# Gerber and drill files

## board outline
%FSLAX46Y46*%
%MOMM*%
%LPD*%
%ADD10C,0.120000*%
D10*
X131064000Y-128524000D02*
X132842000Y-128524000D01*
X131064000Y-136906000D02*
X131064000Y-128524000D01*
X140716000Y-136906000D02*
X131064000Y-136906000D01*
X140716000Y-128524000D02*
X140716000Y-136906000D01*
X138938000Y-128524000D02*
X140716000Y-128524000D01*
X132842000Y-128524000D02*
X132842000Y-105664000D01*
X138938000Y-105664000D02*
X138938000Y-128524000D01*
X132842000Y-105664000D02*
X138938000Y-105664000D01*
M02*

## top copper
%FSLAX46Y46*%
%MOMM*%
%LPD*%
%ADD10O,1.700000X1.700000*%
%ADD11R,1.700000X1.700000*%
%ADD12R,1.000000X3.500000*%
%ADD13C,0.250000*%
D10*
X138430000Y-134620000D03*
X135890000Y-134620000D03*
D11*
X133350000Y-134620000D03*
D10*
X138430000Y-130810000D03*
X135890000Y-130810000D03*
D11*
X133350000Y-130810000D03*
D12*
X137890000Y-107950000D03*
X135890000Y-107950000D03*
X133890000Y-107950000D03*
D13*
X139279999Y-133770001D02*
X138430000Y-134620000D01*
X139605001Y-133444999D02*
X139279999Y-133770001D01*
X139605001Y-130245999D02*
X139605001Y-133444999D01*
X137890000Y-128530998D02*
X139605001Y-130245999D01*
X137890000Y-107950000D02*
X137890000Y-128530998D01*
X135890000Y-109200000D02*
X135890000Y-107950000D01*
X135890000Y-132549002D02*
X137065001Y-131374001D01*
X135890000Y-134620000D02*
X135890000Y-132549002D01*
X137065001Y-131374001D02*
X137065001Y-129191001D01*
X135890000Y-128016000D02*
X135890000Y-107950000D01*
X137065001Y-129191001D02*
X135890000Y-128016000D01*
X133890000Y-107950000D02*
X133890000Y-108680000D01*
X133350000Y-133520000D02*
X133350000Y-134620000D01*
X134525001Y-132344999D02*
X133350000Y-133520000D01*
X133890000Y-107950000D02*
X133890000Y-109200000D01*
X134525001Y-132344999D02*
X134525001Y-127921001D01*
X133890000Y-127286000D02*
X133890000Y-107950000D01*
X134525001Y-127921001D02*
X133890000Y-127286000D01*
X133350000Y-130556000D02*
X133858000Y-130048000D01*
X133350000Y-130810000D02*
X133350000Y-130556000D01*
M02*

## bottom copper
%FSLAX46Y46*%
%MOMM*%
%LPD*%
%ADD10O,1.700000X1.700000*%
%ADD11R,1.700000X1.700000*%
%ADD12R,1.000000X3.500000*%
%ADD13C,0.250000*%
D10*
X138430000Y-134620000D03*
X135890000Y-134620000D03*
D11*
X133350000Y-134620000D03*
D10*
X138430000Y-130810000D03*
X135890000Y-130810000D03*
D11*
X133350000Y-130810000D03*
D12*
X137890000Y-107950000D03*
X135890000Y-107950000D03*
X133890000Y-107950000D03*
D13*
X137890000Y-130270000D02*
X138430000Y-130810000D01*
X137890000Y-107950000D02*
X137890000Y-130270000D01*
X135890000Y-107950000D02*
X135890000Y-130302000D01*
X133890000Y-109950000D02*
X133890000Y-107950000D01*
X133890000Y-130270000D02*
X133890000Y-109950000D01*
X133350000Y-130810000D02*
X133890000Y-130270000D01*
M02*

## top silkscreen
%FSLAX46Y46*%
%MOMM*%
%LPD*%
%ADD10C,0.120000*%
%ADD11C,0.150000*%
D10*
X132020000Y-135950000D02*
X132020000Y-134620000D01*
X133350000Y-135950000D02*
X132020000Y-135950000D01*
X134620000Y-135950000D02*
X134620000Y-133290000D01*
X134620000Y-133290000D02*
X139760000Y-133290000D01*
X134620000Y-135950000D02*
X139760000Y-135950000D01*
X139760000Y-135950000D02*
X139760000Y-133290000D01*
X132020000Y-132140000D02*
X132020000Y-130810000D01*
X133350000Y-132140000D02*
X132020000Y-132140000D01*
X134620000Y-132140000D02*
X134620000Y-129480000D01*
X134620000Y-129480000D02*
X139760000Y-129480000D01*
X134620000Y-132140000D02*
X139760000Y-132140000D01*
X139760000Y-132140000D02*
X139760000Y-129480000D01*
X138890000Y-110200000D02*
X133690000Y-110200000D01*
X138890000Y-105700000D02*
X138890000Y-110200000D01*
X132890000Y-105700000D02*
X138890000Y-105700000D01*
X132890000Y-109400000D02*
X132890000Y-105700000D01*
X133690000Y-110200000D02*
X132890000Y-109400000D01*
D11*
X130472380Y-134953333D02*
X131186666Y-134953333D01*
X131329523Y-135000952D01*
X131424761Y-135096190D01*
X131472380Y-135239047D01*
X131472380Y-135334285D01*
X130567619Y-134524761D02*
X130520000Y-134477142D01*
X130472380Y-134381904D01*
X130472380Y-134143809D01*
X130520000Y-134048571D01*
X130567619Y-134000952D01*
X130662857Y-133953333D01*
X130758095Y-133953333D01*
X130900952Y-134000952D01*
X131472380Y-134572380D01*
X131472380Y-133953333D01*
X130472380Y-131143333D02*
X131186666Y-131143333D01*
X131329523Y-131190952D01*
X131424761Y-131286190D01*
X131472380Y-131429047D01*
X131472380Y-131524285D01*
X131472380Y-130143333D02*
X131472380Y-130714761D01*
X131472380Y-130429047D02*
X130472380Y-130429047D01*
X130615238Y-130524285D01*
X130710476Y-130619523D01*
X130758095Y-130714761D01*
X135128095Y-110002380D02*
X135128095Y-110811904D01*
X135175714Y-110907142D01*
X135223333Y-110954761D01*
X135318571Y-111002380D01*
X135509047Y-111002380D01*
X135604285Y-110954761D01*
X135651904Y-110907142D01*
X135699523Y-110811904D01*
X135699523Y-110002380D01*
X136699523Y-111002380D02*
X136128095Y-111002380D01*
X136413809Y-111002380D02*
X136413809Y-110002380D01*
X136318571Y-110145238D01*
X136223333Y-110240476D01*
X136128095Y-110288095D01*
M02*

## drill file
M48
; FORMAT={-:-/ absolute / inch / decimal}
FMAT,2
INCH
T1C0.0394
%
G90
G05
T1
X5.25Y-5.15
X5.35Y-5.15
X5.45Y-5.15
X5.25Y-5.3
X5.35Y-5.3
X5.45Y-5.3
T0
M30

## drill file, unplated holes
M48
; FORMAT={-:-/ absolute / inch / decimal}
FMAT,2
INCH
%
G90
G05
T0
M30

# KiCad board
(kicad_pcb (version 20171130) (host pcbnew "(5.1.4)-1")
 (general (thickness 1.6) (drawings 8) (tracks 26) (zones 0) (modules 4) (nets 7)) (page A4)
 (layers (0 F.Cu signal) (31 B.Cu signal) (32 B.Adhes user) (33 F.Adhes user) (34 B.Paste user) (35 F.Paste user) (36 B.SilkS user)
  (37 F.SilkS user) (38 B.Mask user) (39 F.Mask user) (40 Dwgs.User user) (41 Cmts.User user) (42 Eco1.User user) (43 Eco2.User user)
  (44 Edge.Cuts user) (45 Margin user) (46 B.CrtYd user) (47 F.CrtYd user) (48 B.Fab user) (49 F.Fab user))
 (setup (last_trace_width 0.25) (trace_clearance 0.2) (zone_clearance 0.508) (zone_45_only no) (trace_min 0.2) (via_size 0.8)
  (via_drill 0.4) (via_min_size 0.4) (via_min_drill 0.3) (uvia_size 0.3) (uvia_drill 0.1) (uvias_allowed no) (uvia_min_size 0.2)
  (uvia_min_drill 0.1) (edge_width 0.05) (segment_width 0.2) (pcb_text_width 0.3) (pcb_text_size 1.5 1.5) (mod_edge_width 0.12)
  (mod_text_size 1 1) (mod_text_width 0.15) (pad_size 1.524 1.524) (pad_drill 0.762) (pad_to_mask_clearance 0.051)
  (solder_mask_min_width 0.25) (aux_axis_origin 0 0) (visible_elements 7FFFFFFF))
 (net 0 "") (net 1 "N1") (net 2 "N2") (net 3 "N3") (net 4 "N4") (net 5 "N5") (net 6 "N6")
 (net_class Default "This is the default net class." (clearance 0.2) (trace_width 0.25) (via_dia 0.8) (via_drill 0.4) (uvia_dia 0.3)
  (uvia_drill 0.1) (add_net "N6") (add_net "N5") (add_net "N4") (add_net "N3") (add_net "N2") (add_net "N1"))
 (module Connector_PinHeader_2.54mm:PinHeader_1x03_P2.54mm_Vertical (layer F.Cu) (at 133.35 134.62 90)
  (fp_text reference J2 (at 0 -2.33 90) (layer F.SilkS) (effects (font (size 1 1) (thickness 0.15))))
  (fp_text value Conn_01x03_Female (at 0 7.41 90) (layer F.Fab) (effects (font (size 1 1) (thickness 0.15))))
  (fp_line (start -1.33 -1.33) (end 0 -1.33) (layer F.SilkS) (width 0.12))
  (fp_line (start -1.33 0) (end -1.33 -1.33) (layer F.SilkS) (width 0.12))
  (fp_line (start -1.33 1.27) (end 1.33 1.27) (layer F.SilkS) (width 0.12))
  (fp_line (start 1.33 1.27) (end 1.33 6.41) (layer F.SilkS) (width 0.12))
  (fp_line (start -1.33 1.27) (end -1.33 6.41) (layer F.SilkS) (width 0.12))
  (fp_line (start -1.33 6.41) (end 1.33 6.41) (layer F.SilkS) (width 0.12))
  (pad 3 thru_hole oval (at 0 5.08 90) (size 1.7 1.7) (drill 1) (layers *.Cu *.Mask) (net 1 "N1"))
  (pad 2 thru_hole oval (at 0 2.54 90) (size 1.7 1.7) (drill 1) (layers *.Cu *.Mask) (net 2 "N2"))
  (pad 1 thru_hole rect (at 0 0 90) (size 1.7 1.7) (drill 1) (layers *.Cu *.Mask) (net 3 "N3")))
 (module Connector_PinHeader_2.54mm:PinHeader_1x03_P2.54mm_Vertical (layer F.Cu) (at 133.35 130.81 90)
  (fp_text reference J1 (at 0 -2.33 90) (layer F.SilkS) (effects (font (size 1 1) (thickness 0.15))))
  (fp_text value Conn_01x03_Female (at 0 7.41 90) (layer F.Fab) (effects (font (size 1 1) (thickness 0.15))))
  (fp_line (start -1.33 -1.33) (end 0 -1.33) (layer F.SilkS) (width 0.12))
  (fp_line (start -1.33 0) (end -1.33 -1.33) (layer F.SilkS) (width 0.12))
  (fp_line (start -1.33 1.27) (end 1.33 1.27) (layer F.SilkS) (width 0.12))
  (fp_line (start 1.33 1.27) (end 1.33 6.41) (layer F.SilkS) (width 0.12))
  (fp_line (start -1.33 1.27) (end -1.33 6.41) (layer F.SilkS) (width 0.12))
  (fp_line (start -1.33 6.41) (end 1.33 6.41) (layer F.SilkS) (width 0.12))
  (pad 3 thru_hole oval (at 0 5.08 90) (size 1.7 1.7) (drill 1) (layers *.Cu *.Mask) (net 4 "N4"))
  (pad 2 thru_hole oval (at 0 2.54 90) (size 1.7 1.7) (drill 1) (layers *.Cu *.Mask) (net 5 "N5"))
  (pad 1 thru_hole rect (at 0 0 90) (size 1.7 1.7) (drill 1) (layers *.Cu *.Mask) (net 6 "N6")))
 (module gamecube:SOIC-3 (layer B.Cu) (at 135.89 107.95)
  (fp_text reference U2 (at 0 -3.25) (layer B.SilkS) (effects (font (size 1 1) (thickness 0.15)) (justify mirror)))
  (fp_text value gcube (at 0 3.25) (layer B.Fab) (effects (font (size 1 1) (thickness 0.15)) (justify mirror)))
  (pad 3 smd rect (at 2 0) (size 1 3.5) (layers B.Cu B.Paste B.Mask) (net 4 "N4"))
  (pad 2 smd rect (at 0 0) (size 1 3.5) (layers B.Cu B.Paste B.Mask) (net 5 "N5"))
  (pad 1 smd rect (at -2 0) (size 1 3.5) (layers B.Cu B.Paste B.Mask) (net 6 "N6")))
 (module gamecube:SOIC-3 (layer F.Cu) (at 135.89 107.95)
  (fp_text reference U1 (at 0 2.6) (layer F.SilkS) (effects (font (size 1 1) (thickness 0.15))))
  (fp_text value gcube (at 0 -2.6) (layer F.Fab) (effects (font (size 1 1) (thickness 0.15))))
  (fp_line (start 3 2.25) (end -2.2 2.25) (layer F.SilkS) (width 0.12))
  (fp_line (start 3 -2.25) (end 3 2.25) (layer F.SilkS) (width 0.12))
  (fp_line (start -3 -2.25) (end 3 -2.25) (layer F.SilkS) (width 0.12))
  (fp_line (start -3 1.45) (end -3 -2.25) (layer F.SilkS) (width 0.12))
  (fp_line (start -2.2 2.25) (end -3 1.45) (layer F.SilkS) (width 0.12))
  (pad 3 smd rect (at 2 0) (size 1 3.5) (layers F.Cu F.Paste F.Mask) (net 1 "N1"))
  (pad 2 smd rect (at 0 0) (size 1 3.5) (layers F.Cu F.Paste F.Mask) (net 2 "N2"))
  (pad 1 smd rect (at -2 0) (size 1 3.5) (layers F.Cu F.Paste F.Mask) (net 3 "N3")))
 (gr_line (start 131.064 128.524) (end 132.842 128.524) (layer Edge.Cuts) (width 0.12))
 (gr_line (start 131.064 136.906) (end 131.064 128.524) (layer Edge.Cuts) (width 0.12))
 (gr_line (start 140.716 136.906) (end 131.064 136.906) (layer Edge.Cuts) (width 0.12))
 (gr_line (start 140.716 128.524) (end 140.716 136.906) (layer Edge.Cuts) (width 0.12))
 (gr_line (start 138.938 128.524) (end 140.716 128.524) (layer Edge.Cuts) (width 0.12))
 (gr_line (start 132.842 128.524) (end 132.842 105.664) (layer Edge.Cuts) (width 0.12))
 (gr_line (start 138.938 105.664) (end 138.938 128.524) (layer Edge.Cuts) (width 0.12))
 (gr_line (start 132.842 105.664) (end 138.938 105.664) (layer Edge.Cuts) (width 0.12))
 (segment (start 139.279999 133.770001) (end 138.43 134.62) (width 0.25) (layer F.Cu) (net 1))
 (segment (start 139.605001 133.444999) (end 139.279999 133.770001) (width 0.25) (layer F.Cu) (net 1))
 (segment (start 139.605001 130.245999) (end 139.605001 133.444999) (width 0.25) (layer F.Cu) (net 1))
 (segment (start 137.89 128.530998) (end 139.605001 130.245999) (width 0.25) (layer F.Cu) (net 1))
 (segment (start 137.89 107.95) (end 137.89 128.530998) (width 0.25) (layer F.Cu) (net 1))
 (segment (start 135.89 109.2) (end 135.89 107.95) (width 0.25) (layer F.Cu) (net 2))
 (segment (start 135.89 132.549002) (end 137.065001 131.374001) (width 0.25) (layer F.Cu) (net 2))
 (segment (start 135.89 134.62) (end 135.89 132.549002) (width 0.25) (layer F.Cu) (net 2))
 (segment (start 137.065001 131.374001) (end 137.065001 129.191001) (width 0.25) (layer F.Cu) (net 2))
 (segment (start 135.89 128.016) (end 135.89 107.95) (width 0.25) (layer F.Cu) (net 2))
 (segment (start 137.065001 129.191001) (end 135.89 128.016) (width 0.25) (layer F.Cu) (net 2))
 (segment (start 133.89 107.95) (end 133.89 108.68) (width 0.25) (layer F.Cu) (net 3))
 (segment (start 133.35 133.52) (end 133.35 134.62) (width 0.25) (layer F.Cu) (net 3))
 (segment (start 134.525001 132.344999) (end 133.35 133.52) (width 0.25) (layer F.Cu) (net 3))
 (segment (start 133.89 107.95) (end 133.89 109.2) (width 0.25) (layer F.Cu) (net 3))
 (segment (start 134.525001 132.344999) (end 134.525001 127.921001) (width 0.25) (layer F.Cu) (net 3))
 (segment (start 133.89 127.286) (end 133.89 107.95) (width 0.25) (layer F.Cu) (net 3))
 (segment (start 134.525001 127.921001) (end 133.89 127.286) (width 0.25) (layer F.Cu) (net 3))
 (segment (start 137.89 130.27) (end 138.43 130.81) (width 0.25) (layer B.Cu) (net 4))
 (segment (start 137.89 107.95) (end 137.89 130.27) (width 0.25) (layer B.Cu) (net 4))
 (segment (start 135.89 107.95) (end 135.89 130.302) (width 0.25) (layer B.Cu) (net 5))
 (segment (start 133.35 130.556) (end 133.858 130.048) (width 0.25) (layer F.Cu) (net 6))
 (segment (start 133.35 130.81) (end 133.35 130.556) (width 0.25) (layer F.Cu) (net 6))
 (segment (start 133.89 109.95) (end 133.89 107.95) (width 0.25) (layer B.Cu) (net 6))
 (segment (start 133.89 130.27) (end 133.89 109.95) (width 0.25) (layer B.Cu) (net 6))
 (segment (start 133.35 130.81) (end 133.89 130.27) (width 0.25) (layer B.Cu) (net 6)))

